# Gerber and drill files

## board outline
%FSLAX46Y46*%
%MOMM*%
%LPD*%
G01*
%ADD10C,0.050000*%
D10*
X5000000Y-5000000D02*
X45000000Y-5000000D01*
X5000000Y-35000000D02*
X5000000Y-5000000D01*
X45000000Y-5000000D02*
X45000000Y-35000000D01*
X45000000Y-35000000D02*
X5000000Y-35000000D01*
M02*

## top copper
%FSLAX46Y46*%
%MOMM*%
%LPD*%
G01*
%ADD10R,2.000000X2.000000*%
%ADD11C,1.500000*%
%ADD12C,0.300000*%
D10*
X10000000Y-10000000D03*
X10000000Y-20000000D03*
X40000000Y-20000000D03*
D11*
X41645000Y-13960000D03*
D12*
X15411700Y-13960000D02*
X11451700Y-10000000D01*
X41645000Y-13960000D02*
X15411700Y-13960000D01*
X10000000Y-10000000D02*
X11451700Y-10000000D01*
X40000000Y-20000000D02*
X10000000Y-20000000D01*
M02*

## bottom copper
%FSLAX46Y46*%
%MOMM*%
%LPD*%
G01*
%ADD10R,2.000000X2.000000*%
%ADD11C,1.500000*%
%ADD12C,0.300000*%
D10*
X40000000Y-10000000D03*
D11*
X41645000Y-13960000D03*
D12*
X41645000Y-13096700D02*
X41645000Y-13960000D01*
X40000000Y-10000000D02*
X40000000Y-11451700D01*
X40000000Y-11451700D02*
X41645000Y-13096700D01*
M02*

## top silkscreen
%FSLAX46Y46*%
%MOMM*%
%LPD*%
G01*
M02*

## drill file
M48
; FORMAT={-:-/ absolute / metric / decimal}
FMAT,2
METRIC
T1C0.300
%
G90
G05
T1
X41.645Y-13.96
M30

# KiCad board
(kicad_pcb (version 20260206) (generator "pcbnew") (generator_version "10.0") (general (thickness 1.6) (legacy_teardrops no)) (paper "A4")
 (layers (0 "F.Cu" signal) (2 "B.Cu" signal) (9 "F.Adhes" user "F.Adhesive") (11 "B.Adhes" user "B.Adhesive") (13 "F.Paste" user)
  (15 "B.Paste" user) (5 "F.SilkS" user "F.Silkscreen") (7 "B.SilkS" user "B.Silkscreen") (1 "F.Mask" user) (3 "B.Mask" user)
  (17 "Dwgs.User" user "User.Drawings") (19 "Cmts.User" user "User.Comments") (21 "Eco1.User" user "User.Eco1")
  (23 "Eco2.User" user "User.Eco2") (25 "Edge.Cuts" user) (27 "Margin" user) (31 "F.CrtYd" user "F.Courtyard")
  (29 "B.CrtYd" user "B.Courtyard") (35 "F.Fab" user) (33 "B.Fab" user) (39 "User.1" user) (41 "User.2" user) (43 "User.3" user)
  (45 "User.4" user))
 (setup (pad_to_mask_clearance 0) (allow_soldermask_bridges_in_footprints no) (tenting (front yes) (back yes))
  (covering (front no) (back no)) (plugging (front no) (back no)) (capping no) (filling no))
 (gr_line (start 5 5) (end 45 5) (stroke (width 0.05) (type default)) (layer "Edge.Cuts"))
 (gr_line (start 5 35) (end 5 5) (stroke (width 0.05) (type default)) (layer "Edge.Cuts"))
 (gr_line (start 45 5) (end 45 35) (stroke (width 0.05) (type default)) (layer "Edge.Cuts"))
 (gr_line (start 45 35) (end 5 35) (stroke (width 0.05) (type default)) (layer "Edge.Cuts"))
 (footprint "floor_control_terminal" (layer "F.Cu") (at 10 10)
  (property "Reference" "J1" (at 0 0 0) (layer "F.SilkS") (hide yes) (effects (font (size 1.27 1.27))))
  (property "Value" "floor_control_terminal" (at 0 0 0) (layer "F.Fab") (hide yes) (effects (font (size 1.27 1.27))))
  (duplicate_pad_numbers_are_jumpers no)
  (pad "1" smd rect (at 0 0) (size 2 2) (layers "F.Cu" "F.Paste" "F.Mask") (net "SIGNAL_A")))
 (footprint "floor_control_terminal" (layer "B.Cu") (at 40 10)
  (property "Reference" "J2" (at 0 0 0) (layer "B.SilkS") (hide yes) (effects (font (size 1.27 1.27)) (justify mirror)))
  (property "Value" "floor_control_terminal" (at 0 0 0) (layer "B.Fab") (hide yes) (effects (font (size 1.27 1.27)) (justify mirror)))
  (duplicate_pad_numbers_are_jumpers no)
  (pad "1" smd rect (at 0 0) (size 2 2) (layers "B.Cu" "B.Paste" "B.Mask") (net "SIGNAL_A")))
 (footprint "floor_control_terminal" (layer "F.Cu") (at 10 20)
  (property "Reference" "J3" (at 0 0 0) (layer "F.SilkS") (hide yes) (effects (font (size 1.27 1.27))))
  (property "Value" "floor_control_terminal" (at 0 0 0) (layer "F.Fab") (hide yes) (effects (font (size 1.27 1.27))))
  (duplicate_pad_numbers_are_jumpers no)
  (pad "1" smd rect (at 0 0) (size 2 2) (layers "F.Cu" "F.Paste" "F.Mask") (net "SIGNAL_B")))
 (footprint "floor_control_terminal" (layer "F.Cu") (at 40 20)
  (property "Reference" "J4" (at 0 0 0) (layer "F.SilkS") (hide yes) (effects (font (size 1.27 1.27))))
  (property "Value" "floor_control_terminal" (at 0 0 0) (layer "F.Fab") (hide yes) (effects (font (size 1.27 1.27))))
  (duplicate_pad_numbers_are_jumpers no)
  (pad "1" smd rect (at 0 0) (size 2 2) (layers "F.Cu" "F.Paste" "F.Mask") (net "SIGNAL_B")))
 (segment (start 15.4117 13.96) (end 11.4517 10) (width 0.3) (layer "F.Cu") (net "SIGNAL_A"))
 (segment (start 41.645 13.96) (end 15.4117 13.96) (width 0.3) (layer "F.Cu") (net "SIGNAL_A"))
 (segment (start 10 10) (end 11.4517 10) (width 0.3) (layer "F.Cu") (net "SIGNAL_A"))
 (via (at 41.645 13.96) (size 1.5) (drill 0.3) (layers "F.Cu" "B.Cu") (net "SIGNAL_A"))
 (segment (start 41.645 13.0967) (end 41.645 13.96) (width 0.3) (layer "B.Cu") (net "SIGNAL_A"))
 (segment (start 40 10) (end 40 11.4517) (width 0.3) (layer "B.Cu") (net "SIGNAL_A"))
 (segment (start 40 11.4517) (end 41.645 13.0967) (width 0.3) (layer "B.Cu") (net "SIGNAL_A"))
 (segment (start 40 20) (end 10 20) (width 0.3) (layer "F.Cu") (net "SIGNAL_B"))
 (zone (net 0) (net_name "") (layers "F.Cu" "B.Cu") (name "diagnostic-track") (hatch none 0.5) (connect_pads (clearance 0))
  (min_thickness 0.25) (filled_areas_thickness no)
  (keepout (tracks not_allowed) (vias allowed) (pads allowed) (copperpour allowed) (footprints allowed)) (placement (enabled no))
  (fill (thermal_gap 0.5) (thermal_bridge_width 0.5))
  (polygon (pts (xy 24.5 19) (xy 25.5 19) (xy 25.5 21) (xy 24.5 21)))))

